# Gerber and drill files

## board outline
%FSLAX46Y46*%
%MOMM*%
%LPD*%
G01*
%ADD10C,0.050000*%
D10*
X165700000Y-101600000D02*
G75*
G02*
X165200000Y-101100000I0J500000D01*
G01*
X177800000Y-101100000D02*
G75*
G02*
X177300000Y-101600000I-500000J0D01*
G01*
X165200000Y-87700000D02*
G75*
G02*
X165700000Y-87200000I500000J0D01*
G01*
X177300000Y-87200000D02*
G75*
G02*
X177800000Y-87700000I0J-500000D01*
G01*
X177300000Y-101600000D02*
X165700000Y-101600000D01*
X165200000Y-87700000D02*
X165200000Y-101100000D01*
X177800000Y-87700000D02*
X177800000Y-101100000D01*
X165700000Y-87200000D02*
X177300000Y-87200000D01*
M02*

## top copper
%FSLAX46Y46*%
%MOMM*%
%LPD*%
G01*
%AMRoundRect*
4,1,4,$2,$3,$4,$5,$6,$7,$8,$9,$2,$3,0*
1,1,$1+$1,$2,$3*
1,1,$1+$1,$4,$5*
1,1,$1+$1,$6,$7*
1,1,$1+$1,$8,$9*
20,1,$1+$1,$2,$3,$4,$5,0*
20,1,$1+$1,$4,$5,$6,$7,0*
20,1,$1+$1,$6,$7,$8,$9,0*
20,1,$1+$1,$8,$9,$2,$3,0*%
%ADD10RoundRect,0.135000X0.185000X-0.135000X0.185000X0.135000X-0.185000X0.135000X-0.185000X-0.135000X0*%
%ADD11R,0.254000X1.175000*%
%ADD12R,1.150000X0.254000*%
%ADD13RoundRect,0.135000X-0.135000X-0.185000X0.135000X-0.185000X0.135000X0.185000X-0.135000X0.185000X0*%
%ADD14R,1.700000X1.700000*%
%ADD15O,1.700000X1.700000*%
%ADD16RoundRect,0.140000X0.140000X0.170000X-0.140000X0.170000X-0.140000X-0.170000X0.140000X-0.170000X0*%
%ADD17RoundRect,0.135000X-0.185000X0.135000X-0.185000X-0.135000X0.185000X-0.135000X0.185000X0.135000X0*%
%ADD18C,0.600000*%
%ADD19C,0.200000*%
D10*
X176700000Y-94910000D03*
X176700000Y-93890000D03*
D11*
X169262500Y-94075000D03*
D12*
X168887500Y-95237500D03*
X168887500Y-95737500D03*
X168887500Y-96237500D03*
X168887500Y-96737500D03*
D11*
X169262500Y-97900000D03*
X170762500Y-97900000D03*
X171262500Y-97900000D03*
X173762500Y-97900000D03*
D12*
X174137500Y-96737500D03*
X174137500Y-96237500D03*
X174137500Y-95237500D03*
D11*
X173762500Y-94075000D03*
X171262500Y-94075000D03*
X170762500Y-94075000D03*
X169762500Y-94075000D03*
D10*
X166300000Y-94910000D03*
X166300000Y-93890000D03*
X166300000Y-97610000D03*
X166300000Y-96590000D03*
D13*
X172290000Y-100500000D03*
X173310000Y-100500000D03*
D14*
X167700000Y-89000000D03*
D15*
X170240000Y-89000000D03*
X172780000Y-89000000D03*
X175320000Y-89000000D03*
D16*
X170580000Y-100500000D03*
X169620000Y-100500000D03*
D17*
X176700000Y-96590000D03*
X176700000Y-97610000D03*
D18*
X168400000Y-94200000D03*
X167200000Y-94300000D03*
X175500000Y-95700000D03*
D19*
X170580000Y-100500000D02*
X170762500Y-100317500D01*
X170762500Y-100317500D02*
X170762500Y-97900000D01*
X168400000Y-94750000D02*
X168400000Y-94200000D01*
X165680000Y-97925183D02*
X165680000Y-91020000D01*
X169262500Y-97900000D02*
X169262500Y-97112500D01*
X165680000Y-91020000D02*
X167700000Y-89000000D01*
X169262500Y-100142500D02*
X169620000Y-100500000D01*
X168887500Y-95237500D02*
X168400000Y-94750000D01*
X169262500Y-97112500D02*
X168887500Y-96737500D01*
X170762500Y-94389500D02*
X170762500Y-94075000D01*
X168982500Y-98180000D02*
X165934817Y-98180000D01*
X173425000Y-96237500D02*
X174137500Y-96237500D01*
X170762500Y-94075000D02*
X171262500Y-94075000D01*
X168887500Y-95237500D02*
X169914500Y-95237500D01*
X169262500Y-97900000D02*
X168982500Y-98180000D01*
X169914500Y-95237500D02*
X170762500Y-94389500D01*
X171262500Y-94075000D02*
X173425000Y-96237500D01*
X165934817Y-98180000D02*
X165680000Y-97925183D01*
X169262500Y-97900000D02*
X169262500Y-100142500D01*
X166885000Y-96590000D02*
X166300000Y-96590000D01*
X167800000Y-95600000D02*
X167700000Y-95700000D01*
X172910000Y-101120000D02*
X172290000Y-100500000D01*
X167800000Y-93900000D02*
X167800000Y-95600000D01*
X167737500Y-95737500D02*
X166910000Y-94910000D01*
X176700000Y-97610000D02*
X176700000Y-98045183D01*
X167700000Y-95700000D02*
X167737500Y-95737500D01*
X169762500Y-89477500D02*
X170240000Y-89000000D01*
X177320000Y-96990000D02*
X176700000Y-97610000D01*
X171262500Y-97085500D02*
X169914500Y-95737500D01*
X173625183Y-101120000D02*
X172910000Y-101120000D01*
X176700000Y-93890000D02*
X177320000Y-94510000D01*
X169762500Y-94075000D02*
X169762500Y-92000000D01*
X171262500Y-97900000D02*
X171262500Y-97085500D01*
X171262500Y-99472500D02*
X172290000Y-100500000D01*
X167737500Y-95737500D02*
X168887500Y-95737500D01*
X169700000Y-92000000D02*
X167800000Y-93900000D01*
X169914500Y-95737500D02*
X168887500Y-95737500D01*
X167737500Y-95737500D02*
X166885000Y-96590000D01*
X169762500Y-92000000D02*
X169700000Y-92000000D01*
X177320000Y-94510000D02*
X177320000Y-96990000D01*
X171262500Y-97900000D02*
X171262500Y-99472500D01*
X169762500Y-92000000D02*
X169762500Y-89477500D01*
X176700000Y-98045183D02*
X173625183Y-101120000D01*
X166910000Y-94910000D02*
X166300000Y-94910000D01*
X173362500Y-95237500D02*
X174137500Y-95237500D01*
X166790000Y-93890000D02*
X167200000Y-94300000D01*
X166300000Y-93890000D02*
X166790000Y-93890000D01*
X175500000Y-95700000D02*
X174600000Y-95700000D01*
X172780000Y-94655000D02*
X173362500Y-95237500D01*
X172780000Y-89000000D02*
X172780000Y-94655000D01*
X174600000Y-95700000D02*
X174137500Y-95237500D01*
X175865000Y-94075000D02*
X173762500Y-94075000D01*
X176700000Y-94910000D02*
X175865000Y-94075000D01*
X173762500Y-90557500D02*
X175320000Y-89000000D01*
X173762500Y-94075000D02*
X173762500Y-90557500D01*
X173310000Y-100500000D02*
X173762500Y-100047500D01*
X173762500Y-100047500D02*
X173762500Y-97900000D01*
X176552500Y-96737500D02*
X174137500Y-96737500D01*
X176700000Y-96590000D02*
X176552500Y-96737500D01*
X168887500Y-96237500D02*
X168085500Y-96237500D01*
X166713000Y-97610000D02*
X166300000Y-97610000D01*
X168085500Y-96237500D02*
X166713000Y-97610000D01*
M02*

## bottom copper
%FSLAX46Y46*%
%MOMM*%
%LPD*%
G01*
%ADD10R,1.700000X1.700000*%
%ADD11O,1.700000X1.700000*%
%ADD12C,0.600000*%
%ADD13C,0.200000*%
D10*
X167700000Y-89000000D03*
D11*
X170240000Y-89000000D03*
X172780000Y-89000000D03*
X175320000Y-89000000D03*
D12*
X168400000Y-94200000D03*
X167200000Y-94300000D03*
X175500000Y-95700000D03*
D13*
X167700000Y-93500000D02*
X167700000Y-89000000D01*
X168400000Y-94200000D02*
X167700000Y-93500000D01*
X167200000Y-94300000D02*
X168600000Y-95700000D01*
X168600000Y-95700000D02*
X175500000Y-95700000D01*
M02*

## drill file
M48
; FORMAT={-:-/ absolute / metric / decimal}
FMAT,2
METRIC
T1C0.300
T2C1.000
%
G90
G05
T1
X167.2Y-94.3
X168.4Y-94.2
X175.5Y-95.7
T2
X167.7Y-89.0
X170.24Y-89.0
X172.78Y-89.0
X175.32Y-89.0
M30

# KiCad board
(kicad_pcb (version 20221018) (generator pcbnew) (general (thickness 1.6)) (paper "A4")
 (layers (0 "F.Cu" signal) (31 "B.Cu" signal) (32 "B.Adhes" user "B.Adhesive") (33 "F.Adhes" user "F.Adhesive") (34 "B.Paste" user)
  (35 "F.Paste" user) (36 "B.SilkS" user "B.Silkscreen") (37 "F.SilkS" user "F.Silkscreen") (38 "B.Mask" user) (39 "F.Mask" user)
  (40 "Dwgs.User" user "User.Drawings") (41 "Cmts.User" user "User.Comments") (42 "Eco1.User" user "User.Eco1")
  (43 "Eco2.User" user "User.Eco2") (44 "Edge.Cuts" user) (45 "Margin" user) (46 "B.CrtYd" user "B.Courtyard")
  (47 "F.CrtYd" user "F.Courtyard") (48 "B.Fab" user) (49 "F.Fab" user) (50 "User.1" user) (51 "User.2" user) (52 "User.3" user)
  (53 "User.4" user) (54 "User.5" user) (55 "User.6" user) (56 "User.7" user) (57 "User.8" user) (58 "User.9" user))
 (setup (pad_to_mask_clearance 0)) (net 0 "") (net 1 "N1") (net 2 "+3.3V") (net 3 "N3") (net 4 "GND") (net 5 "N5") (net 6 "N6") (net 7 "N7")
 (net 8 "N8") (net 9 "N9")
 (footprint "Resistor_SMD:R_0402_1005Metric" (layer "F.Cu") (at 176.7 94.4 90)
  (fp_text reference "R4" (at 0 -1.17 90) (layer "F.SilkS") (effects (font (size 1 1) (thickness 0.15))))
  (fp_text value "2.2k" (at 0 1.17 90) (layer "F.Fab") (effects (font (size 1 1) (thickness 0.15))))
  (pad "1" smd roundrect (at -0.51 0 90) (size 0.54 0.64) (layers "F.Cu" "F.Paste" "F.Mask") (roundrect_rratio 0.25) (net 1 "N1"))
  (pad "2" smd roundrect (at 0.51 0 90) (size 0.54 0.64) (layers "F.Cu" "F.Paste" "F.Mask") (roundrect_rratio 0.25) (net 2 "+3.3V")))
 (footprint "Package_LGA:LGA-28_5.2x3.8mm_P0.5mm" (layer "F.Cu") (at 171.5125 95.9875)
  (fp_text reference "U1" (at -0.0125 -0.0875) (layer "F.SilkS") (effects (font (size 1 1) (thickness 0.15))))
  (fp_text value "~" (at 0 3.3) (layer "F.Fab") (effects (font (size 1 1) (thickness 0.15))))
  (pad "1" smd rect (at -2.25 -1.9125) (size 0.254 1.175) (layers "F.Cu" "F.Paste" "F.Mask") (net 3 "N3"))
  (pad "2" smd rect (at -2.625 -0.75 90) (size 0.254 1.15) (layers "F.Cu" "F.Paste" "F.Mask") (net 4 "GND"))
  (pad "3" smd rect (at -2.625 -0.25 90) (size 0.254 1.15) (layers "F.Cu" "F.Paste" "F.Mask") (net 2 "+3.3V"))
  (pad "4" smd rect (at -2.625 0.25 90) (size 0.254 1.15) (layers "F.Cu" "F.Paste" "F.Mask") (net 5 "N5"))
  (pad "5" smd rect (at -2.625 0.75 90) (size 0.254 1.15) (layers "F.Cu" "F.Paste" "F.Mask") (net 4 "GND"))
  (pad "6" smd rect (at -2.25 1.9125) (size 0.254 1.175) (layers "F.Cu" "F.Paste" "F.Mask") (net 4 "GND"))
  (pad "9" smd rect (at -0.75 1.9125) (size 0.254 1.175) (layers "F.Cu" "F.Paste" "F.Mask") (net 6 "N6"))
  (pad "10" smd rect (at -0.25 1.9125) (size 0.254 1.175) (layers "F.Cu" "F.Paste" "F.Mask") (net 2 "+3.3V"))
  (pad "15" smd rect (at 2.25 1.9125) (size 0.254 1.175) (layers "F.Cu" "F.Paste" "F.Mask") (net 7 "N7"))
  (pad "16" smd rect (at 2.625 0.75 90) (size 0.254 1.15) (layers "F.Cu" "F.Paste" "F.Mask") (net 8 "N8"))
  (pad "17" smd rect (at 2.625 0.25 90) (size 0.254 1.15) (layers "F.Cu" "F.Paste" "F.Mask") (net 4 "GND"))
  (pad "19" smd rect (at 2.625 -0.75 90) (size 0.254 1.15) (layers "F.Cu" "F.Paste" "F.Mask") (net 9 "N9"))
  (pad "20" smd rect (at 2.25 -1.9125) (size 0.254 1.175) (layers "F.Cu" "F.Paste" "F.Mask") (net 1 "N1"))
  (pad "25" smd rect (at -0.25 -1.9125) (size 0.254 1.175) (layers "F.Cu" "F.Paste" "F.Mask") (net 4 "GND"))
  (pad "26" smd rect (at -0.75 -1.9125) (size 0.254 1.175) (layers "F.Cu" "F.Paste" "F.Mask") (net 4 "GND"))
  (pad "28" smd rect (at -1.75 -1.9125) (size 0.254 1.175) (layers "F.Cu" "F.Paste" "F.Mask") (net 2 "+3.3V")))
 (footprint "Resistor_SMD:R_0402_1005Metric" (layer "F.Cu") (at 166.3 94.4 90)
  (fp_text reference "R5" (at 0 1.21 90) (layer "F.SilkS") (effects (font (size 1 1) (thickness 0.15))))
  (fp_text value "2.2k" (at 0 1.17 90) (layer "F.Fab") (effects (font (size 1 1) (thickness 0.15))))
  (pad "1" smd roundrect (at -0.51 0 90) (size 0.54 0.64) (layers "F.Cu" "F.Paste" "F.Mask") (roundrect_rratio 0.25) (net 2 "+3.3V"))
  (pad "2" smd roundrect (at 0.51 0 90) (size 0.54 0.64) (layers "F.Cu" "F.Paste" "F.Mask") (roundrect_rratio 0.25) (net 9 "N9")))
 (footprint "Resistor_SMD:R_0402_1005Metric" (layer "F.Cu") (at 166.3 97.1 90)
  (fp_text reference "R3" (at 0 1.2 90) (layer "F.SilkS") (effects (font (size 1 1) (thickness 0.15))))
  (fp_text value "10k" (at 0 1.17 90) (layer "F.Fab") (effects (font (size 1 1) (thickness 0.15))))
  (pad "1" smd roundrect (at -0.51 0 90) (size 0.54 0.64) (layers "F.Cu" "F.Paste" "F.Mask") (roundrect_rratio 0.25) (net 5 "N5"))
  (pad "2" smd roundrect (at 0.51 0 90) (size 0.54 0.64) (layers "F.Cu" "F.Paste" "F.Mask") (roundrect_rratio 0.25) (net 2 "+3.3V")))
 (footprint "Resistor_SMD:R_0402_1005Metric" (layer "F.Cu") (at 172.8 100.5)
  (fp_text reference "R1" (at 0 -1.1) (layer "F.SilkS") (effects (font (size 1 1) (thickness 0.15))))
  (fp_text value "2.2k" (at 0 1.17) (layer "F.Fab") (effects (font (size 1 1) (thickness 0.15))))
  (pad "1" smd roundrect (at -0.51 0) (size 0.54 0.64) (layers "F.Cu" "F.Paste" "F.Mask") (roundrect_rratio 0.25) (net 2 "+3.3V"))
  (pad "2" smd roundrect (at 0.51 0) (size 0.54 0.64) (layers "F.Cu" "F.Paste" "F.Mask") (roundrect_rratio 0.25) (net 7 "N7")))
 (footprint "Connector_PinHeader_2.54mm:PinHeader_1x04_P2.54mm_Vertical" (layer "F.Cu") (at 167.7 89 90)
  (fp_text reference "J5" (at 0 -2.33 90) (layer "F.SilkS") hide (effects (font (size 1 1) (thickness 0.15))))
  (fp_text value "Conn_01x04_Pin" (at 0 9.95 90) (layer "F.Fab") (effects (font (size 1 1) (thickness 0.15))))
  (pad "1" thru_hole rect (at 0 0 90) (size 1.7 1.7) (drill 1) (layers "*.Cu" "*.Mask") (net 4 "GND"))
  (pad "2" thru_hole oval (at 0 2.54 90) (size 1.7 1.7) (drill 1) (layers "*.Cu" "*.Mask") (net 2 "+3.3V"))
  (pad "3" thru_hole oval (at 0 5.08 90) (size 1.7 1.7) (drill 1) (layers "*.Cu" "*.Mask") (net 9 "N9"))
  (pad "4" thru_hole oval (at 0 7.62 90) (size 1.7 1.7) (drill 1) (layers "*.Cu" "*.Mask") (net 1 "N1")))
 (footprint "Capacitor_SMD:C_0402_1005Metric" (layer "F.Cu") (at 170.1 100.5 180)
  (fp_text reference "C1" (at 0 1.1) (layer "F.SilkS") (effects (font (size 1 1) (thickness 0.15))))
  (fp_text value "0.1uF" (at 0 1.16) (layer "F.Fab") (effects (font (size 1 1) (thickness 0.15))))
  (pad "1" smd roundrect (at -0.48 0 180) (size 0.56 0.62) (layers "F.Cu" "F.Paste" "F.Mask") (roundrect_rratio 0.25) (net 6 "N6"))
  (pad "2" smd roundrect (at 0.48 0 180) (size 0.56 0.62) (layers "F.Cu" "F.Paste" "F.Mask") (roundrect_rratio 0.25) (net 4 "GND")))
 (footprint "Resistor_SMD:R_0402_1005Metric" (layer "F.Cu") (at 176.7 97.1 -90)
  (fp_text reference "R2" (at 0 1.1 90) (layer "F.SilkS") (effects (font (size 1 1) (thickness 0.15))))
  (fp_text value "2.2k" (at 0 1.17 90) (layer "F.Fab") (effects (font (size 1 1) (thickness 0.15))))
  (pad "1" smd roundrect (at -0.51 0 270) (size 0.54 0.64) (layers "F.Cu" "F.Paste" "F.Mask") (roundrect_rratio 0.25) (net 8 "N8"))
  (pad "2" smd roundrect (at 0.51 0 270) (size 0.54 0.64) (layers "F.Cu" "F.Paste" "F.Mask") (roundrect_rratio 0.25) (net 2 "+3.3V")))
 (gr_arc (start 165.7 101.6) (mid 165.346447 101.453553) (end 165.2 101.1) (stroke (width 0.05) (type default)) (layer "Edge.Cuts"))
 (gr_arc (start 177.8 101.1) (mid 177.653553 101.453553) (end 177.3 101.6) (stroke (width 0.05) (type default)) (layer "Edge.Cuts"))
 (gr_arc (start 165.2 87.7) (mid 165.346447 87.346447) (end 165.7 87.2) (stroke (width 0.05) (type default)) (layer "Edge.Cuts"))
 (gr_arc (start 177.3 87.2) (mid 177.653553 87.346447) (end 177.8 87.7) (stroke (width 0.05) (type default)) (layer "Edge.Cuts"))
 (gr_line (start 177.3 101.6) (end 165.7 101.6) (stroke (width 0.05) (type default)) (layer "Edge.Cuts"))
 (gr_line (start 165.2 87.7) (end 165.2 101.1) (stroke (width 0.05) (type default)) (layer "Edge.Cuts"))
 (gr_line (start 177.8 87.7) (end 177.8 101.1) (stroke (width 0.05) (type default)) (layer "Edge.Cuts"))
 (gr_line (start 165.7 87.2) (end 177.3 87.2) (stroke (width 0.05) (type default)) (layer "Edge.Cuts"))
 (segment (start 170.58 100.5) (end 170.7625 100.3175) (width 0.2) (layer "F.Cu") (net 6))
 (segment (start 170.7625 100.3175) (end 170.7625 97.9) (width 0.2) (layer "F.Cu") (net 6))
 (segment (start 168.4 94.75) (end 168.4 94.2) (width 0.2) (layer "F.Cu") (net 4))
 (segment (start 165.68 97.925183) (end 165.68 91.02) (width 0.2) (layer "F.Cu") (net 4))
 (segment (start 169.2625 97.9) (end 169.2625 97.1125) (width 0.2) (layer "F.Cu") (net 4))
 (segment (start 165.68 91.02) (end 167.7 89) (width 0.2) (layer "F.Cu") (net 4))
 (segment (start 169.2625 100.1425) (end 169.62 100.5) (width 0.2) (layer "F.Cu") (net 4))
 (segment (start 168.8875 95.2375) (end 168.4 94.75) (width 0.2) (layer "F.Cu") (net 4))
 (segment (start 169.2625 97.1125) (end 168.8875 96.7375) (width 0.2) (layer "F.Cu") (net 4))
 (segment (start 170.7625 94.3895) (end 170.7625 94.075) (width 0.2) (layer "F.Cu") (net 4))
 (segment (start 168.9825 98.18) (end 165.934817 98.18) (width 0.2) (layer "F.Cu") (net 4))
 (segment (start 173.425 96.2375) (end 174.1375 96.2375) (width 0.2) (layer "F.Cu") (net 4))
 (segment (start 170.7625 94.075) (end 171.2625 94.075) (width 0.2) (layer "F.Cu") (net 4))
 (segment (start 168.8875 95.2375) (end 169.9145 95.2375) (width 0.2) (layer "F.Cu") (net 4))
 (segment (start 169.2625 97.9) (end 168.9825 98.18) (width 0.2) (layer "F.Cu") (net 4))
 (segment (start 169.9145 95.2375) (end 170.7625 94.3895) (width 0.2) (layer "F.Cu") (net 4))
 (segment (start 171.2625 94.075) (end 173.425 96.2375) (width 0.2) (layer "F.Cu") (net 4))
 (segment (start 165.934817 98.18) (end 165.68 97.925183) (width 0.2) (layer "F.Cu") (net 4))
 (segment (start 169.2625 97.9) (end 169.2625 100.1425) (width 0.2) (layer "F.Cu") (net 4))
 (via (at 168.4 94.2) (size 0.6) (drill 0.3) (layers "F.Cu" "B.Cu") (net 4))
 (segment (start 167.7 93.5) (end 167.7 89) (width 0.2) (layer "B.Cu") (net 4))
 (segment (start 168.4 94.2) (end 167.7 93.5) (width 0.2) (layer "B.Cu") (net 4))
 (segment (start 166.885 96.59) (end 166.3 96.59) (width 0.2) (layer "F.Cu") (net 2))
 (segment (start 167.8 95.6) (end 167.7 95.7) (width 0.2) (layer "F.Cu") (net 2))
 (segment (start 172.91 101.12) (end 172.29 100.5) (width 0.2) (layer "F.Cu") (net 2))
 (segment (start 167.8 93.9) (end 167.8 95.6) (width 0.2) (layer "F.Cu") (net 2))
 (segment (start 167.7375 95.7375) (end 166.91 94.91) (width 0.2) (layer "F.Cu") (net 2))
 (segment (start 176.7 97.61) (end 176.7 98.045183) (width 0.2) (layer "F.Cu") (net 2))
 (segment (start 167.7 95.7) (end 167.7375 95.7375) (width 0.2) (layer "F.Cu") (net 2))
 (segment (start 169.7625 89.4775) (end 170.24 89) (width 0.2) (layer "F.Cu") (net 2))
 (segment (start 177.32 96.99) (end 176.7 97.61) (width 0.2) (layer "F.Cu") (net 2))
 (segment (start 171.2625 97.0855) (end 169.9145 95.7375) (width 0.2) (layer "F.Cu") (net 2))
 (segment (start 173.625183 101.12) (end 172.91 101.12) (width 0.2) (layer "F.Cu") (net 2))
 (segment (start 176.7 93.89) (end 177.32 94.51) (width 0.2) (layer "F.Cu") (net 2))
 (segment (start 169.7625 94.075) (end 169.7625 92) (width 0.2) (layer "F.Cu") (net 2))
 (segment (start 171.2625 97.9) (end 171.2625 97.0855) (width 0.2) (layer "F.Cu") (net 2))
 (segment (start 171.2625 99.4725) (end 172.29 100.5) (width 0.2) (layer "F.Cu") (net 2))
 (segment (start 167.7375 95.7375) (end 168.8875 95.7375) (width 0.2) (layer "F.Cu") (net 2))
 (segment (start 169.7 92) (end 167.8 93.9) (width 0.2) (layer "F.Cu") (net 2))
 (segment (start 169.9145 95.7375) (end 168.8875 95.7375) (width 0.2) (layer "F.Cu") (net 2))
 (segment (start 167.7375 95.7375) (end 166.885 96.59) (width 0.2) (layer "F.Cu") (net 2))
 (segment (start 169.7625 92) (end 169.7 92) (width 0.2) (layer "F.Cu") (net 2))
 (segment (start 177.32 94.51) (end 177.32 96.99) (width 0.2) (layer "F.Cu") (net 2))
 (segment (start 171.2625 97.9) (end 171.2625 99.4725) (width 0.2) (layer "F.Cu") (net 2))
 (segment (start 169.7625 92) (end 169.7625 89.4775) (width 0.2) (layer "F.Cu") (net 2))
 (segment (start 176.7 98.045183) (end 173.625183 101.12) (width 0.2) (layer "F.Cu") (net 2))
 (segment (start 166.91 94.91) (end 166.3 94.91) (width 0.2) (layer "F.Cu") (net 2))
 (segment (start 173.3625 95.2375) (end 174.1375 95.2375) (width 0.2) (layer "F.Cu") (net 9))
 (segment (start 166.79 93.89) (end 167.2 94.3) (width 0.2) (layer "F.Cu") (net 9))
 (segment (start 166.3 93.89) (end 166.79 93.89) (width 0.2) (layer "F.Cu") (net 9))
 (segment (start 175.5 95.7) (end 174.6 95.7) (width 0.2) (layer "F.Cu") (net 9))
 (segment (start 172.78 94.655) (end 173.3625 95.2375) (width 0.2) (layer "F.Cu") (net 9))
 (segment (start 172.78 89) (end 172.78 94.655) (width 0.2) (layer "F.Cu") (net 9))
 (segment (start 174.6 95.7) (end 174.1375 95.2375) (width 0.2) (layer "F.Cu") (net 9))
 (via (at 167.2 94.3) (size 0.6) (drill 0.3) (layers "F.Cu" "B.Cu") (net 9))
 (via (at 175.5 95.7) (size 0.6) (drill 0.3) (layers "F.Cu" "B.Cu") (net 9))
 (segment (start 167.2 94.3) (end 168.6 95.7) (width 0.2) (layer "B.Cu") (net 9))
 (segment (start 168.6 95.7) (end 175.5 95.7) (width 0.2) (layer "B.Cu") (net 9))
 (segment (start 175.865 94.075) (end 173.7625 94.075) (width 0.2) (layer "F.Cu") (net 1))
 (segment (start 176.7 94.91) (end 175.865 94.075) (width 0.2) (layer "F.Cu") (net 1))
 (segment (start 173.7625 90.5575) (end 175.32 89) (width 0.2) (layer "F.Cu") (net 1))
 (segment (start 173.7625 94.075) (end 173.7625 90.5575) (width 0.2) (layer "F.Cu") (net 1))
 (segment (start 173.31 100.5) (end 173.7625 100.0475) (width 0.2) (layer "F.Cu") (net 7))
 (segment (start 173.7625 100.0475) (end 173.7625 97.9) (width 0.2) (layer "F.Cu") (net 7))
 (segment (start 176.5525 96.7375) (end 174.1375 96.7375) (width 0.2) (layer "F.Cu") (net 8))
 (segment (start 176.7 96.59) (end 176.5525 96.7375) (width 0.2) (layer "F.Cu") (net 8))
 (segment (start 168.8875 96.2375) (end 168.0855 96.2375) (width 0.2) (layer "F.Cu") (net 5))
 (segment (start 166.713 97.61) (end 166.3 97.61) (width 0.2) (layer "F.Cu") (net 5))
 (segment (start 168.0855 96.2375) (end 166.713 97.61) (width 0.2) (layer "F.Cu") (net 5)))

